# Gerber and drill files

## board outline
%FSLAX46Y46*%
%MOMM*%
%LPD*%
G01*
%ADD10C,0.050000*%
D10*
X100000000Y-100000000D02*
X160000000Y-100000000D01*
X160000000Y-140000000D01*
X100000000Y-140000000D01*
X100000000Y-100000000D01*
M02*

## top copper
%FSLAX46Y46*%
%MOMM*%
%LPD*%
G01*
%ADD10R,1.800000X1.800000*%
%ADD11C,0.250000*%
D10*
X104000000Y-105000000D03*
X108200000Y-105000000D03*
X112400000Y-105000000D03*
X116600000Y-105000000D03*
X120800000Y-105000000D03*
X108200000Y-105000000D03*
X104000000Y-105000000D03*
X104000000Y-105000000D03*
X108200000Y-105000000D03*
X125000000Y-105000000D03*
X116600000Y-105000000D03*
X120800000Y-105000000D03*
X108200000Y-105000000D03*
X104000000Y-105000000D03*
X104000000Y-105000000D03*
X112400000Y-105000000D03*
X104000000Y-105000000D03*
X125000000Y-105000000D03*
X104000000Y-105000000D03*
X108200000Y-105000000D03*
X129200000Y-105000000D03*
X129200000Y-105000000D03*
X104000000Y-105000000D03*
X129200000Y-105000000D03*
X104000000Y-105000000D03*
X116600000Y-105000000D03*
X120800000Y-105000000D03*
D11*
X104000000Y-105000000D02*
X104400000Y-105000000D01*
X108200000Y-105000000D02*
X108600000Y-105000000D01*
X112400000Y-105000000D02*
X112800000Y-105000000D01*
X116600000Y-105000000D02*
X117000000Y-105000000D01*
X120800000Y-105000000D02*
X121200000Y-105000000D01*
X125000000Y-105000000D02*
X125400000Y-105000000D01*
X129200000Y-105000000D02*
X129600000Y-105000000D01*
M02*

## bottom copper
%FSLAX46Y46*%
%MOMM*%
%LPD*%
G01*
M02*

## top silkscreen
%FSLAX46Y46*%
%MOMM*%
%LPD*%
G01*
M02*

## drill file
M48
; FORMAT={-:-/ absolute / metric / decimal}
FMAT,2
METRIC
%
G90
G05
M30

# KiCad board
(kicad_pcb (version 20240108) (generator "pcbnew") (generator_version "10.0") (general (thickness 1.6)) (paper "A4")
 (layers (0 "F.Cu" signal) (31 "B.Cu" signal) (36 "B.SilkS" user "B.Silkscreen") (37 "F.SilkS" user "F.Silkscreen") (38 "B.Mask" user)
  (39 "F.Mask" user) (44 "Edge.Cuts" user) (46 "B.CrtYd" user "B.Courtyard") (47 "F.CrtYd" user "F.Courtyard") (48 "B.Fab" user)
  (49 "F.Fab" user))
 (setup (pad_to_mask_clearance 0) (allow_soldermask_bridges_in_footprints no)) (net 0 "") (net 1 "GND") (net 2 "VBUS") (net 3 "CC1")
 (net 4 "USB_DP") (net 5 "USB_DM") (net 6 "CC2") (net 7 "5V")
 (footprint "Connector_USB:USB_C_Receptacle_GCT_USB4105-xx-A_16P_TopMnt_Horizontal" (layer "F.Cu") (at 100 100)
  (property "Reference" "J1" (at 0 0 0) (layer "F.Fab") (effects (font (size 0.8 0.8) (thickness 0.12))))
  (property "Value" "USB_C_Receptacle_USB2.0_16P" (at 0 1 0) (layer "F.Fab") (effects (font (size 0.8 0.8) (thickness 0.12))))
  (pad "A1" smd rect (at 4.000 5.000) (size 1.8 1.8) (layers "F.Cu" "F.Paste" "F.Mask") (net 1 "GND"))
  (pad "A4" smd rect (at 8.200 5.000) (size 1.8 1.8) (layers "F.Cu" "F.Paste" "F.Mask") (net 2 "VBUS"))
  (pad "A5" smd rect (at 12.400 5.000) (size 1.8 1.8) (layers "F.Cu" "F.Paste" "F.Mask") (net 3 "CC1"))
  (pad "A6" smd rect (at 16.600 5.000) (size 1.8 1.8) (layers "F.Cu" "F.Paste" "F.Mask") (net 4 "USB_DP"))
  (pad "A7" smd rect (at 20.800 5.000) (size 1.8 1.8) (layers "F.Cu" "F.Paste" "F.Mask") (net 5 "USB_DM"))
  (pad "A9" smd rect (at 8.200 5.000) (size 1.8 1.8) (layers "F.Cu" "F.Paste" "F.Mask") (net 2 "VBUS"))
  (pad "A12" smd rect (at 4.000 5.000) (size 1.8 1.8) (layers "F.Cu" "F.Paste" "F.Mask") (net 1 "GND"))
  (pad "B1" smd rect (at 4.000 5.000) (size 1.8 1.8) (layers "F.Cu" "F.Paste" "F.Mask") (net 1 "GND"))
  (pad "B4" smd rect (at 8.200 5.000) (size 1.8 1.8) (layers "F.Cu" "F.Paste" "F.Mask") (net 2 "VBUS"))
  (pad "B5" smd rect (at 25.000 5.000) (size 1.8 1.8) (layers "F.Cu" "F.Paste" "F.Mask") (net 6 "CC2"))
  (pad "B6" smd rect (at 16.600 5.000) (size 1.8 1.8) (layers "F.Cu" "F.Paste" "F.Mask") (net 4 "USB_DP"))
  (pad "B7" smd rect (at 20.800 5.000) (size 1.8 1.8) (layers "F.Cu" "F.Paste" "F.Mask") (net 5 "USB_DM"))
  (pad "B9" smd rect (at 8.200 5.000) (size 1.8 1.8) (layers "F.Cu" "F.Paste" "F.Mask") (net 2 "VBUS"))
  (pad "B12" smd rect (at 4.000 5.000) (size 1.8 1.8) (layers "F.Cu" "F.Paste" "F.Mask") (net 1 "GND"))
  (pad "SH" smd rect (at 4.000 5.000) (size 1.8 1.8) (layers "F.Cu" "F.Paste" "F.Mask") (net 1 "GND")))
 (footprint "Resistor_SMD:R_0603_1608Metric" (layer "F.Cu") (at 100 100)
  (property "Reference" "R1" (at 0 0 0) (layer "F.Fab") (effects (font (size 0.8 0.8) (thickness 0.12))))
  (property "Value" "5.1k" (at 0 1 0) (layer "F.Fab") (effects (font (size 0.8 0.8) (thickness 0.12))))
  (pad "1" smd rect (at 12.400 5.000) (size 1.8 1.8) (layers "F.Cu" "F.Paste" "F.Mask") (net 3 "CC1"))
  (pad "2" smd rect (at 4.000 5.000) (size 1.8 1.8) (layers "F.Cu" "F.Paste" "F.Mask") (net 1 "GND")))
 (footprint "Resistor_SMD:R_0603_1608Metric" (layer "F.Cu") (at 100 100)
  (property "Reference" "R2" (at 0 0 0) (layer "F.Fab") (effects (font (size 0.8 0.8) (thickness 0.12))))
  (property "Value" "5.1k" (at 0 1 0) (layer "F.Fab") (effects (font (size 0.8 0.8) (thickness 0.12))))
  (pad "1" smd rect (at 25.000 5.000) (size 1.8 1.8) (layers "F.Cu" "F.Paste" "F.Mask") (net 6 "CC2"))
  (pad "2" smd rect (at 4.000 5.000) (size 1.8 1.8) (layers "F.Cu" "F.Paste" "F.Mask") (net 1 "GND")))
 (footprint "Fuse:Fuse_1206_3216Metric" (layer "F.Cu") (at 100 100)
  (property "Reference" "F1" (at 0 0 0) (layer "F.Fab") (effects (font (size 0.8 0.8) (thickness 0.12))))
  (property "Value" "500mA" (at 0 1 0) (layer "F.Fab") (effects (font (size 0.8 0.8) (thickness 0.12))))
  (pad "1" smd rect (at 8.200 5.000) (size 1.8 1.8) (layers "F.Cu" "F.Paste" "F.Mask") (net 2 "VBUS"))
  (pad "2" smd rect (at 29.200 5.000) (size 1.8 1.8) (layers "F.Cu" "F.Paste" "F.Mask") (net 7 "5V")))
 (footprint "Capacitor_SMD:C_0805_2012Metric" (layer "F.Cu") (at 100 100)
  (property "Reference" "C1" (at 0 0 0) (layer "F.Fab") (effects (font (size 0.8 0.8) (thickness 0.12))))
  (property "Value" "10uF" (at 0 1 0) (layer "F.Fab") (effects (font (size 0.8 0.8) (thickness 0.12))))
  (pad "1" smd rect (at 29.200 5.000) (size 1.8 1.8) (layers "F.Cu" "F.Paste" "F.Mask") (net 7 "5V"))
  (pad "2" smd rect (at 4.000 5.000) (size 1.8 1.8) (layers "F.Cu" "F.Paste" "F.Mask") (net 1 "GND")))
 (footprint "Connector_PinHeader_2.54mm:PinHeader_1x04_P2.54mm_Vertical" (layer "F.Cu") (at 100 100)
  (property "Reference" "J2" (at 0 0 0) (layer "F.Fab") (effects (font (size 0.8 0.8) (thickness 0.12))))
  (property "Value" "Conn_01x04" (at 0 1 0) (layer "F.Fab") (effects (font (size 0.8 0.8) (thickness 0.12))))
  (pad "1" smd rect (at 29.200 5.000) (size 1.8 1.8) (layers "F.Cu" "F.Paste" "F.Mask") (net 7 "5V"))
  (pad "2" smd rect (at 4.000 5.000) (size 1.8 1.8) (layers "F.Cu" "F.Paste" "F.Mask") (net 1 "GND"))
  (pad "3" smd rect (at 16.600 5.000) (size 1.8 1.8) (layers "F.Cu" "F.Paste" "F.Mask") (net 4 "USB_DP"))
  (pad "4" smd rect (at 20.800 5.000) (size 1.8 1.8) (layers "F.Cu" "F.Paste" "F.Mask") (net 5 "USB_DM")))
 (gr_rect (start 100 100) (end 160 140) (stroke (width 0.05) (type default)) (fill none) (layer "Edge.Cuts"))
 (segment (start 104.000 105.000) (end 104.400 105.000) (width 0.25) (layer "F.Cu") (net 1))
 (segment (start 108.200 105.000) (end 108.600 105.000) (width 0.25) (layer "F.Cu") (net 2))
 (segment (start 112.400 105.000) (end 112.800 105.000) (width 0.25) (layer "F.Cu") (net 3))
 (segment (start 116.600 105.000) (end 117.000 105.000) (width 0.25) (layer "F.Cu") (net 4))
 (segment (start 120.800 105.000) (end 121.200 105.000) (width 0.25) (layer "F.Cu") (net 5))
 (segment (start 125.000 105.000) (end 125.400 105.000) (width 0.25) (layer "F.Cu") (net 6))
 (segment (start 129.200 105.000) (end 129.600 105.000) (width 0.25) (layer "F.Cu") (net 7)))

